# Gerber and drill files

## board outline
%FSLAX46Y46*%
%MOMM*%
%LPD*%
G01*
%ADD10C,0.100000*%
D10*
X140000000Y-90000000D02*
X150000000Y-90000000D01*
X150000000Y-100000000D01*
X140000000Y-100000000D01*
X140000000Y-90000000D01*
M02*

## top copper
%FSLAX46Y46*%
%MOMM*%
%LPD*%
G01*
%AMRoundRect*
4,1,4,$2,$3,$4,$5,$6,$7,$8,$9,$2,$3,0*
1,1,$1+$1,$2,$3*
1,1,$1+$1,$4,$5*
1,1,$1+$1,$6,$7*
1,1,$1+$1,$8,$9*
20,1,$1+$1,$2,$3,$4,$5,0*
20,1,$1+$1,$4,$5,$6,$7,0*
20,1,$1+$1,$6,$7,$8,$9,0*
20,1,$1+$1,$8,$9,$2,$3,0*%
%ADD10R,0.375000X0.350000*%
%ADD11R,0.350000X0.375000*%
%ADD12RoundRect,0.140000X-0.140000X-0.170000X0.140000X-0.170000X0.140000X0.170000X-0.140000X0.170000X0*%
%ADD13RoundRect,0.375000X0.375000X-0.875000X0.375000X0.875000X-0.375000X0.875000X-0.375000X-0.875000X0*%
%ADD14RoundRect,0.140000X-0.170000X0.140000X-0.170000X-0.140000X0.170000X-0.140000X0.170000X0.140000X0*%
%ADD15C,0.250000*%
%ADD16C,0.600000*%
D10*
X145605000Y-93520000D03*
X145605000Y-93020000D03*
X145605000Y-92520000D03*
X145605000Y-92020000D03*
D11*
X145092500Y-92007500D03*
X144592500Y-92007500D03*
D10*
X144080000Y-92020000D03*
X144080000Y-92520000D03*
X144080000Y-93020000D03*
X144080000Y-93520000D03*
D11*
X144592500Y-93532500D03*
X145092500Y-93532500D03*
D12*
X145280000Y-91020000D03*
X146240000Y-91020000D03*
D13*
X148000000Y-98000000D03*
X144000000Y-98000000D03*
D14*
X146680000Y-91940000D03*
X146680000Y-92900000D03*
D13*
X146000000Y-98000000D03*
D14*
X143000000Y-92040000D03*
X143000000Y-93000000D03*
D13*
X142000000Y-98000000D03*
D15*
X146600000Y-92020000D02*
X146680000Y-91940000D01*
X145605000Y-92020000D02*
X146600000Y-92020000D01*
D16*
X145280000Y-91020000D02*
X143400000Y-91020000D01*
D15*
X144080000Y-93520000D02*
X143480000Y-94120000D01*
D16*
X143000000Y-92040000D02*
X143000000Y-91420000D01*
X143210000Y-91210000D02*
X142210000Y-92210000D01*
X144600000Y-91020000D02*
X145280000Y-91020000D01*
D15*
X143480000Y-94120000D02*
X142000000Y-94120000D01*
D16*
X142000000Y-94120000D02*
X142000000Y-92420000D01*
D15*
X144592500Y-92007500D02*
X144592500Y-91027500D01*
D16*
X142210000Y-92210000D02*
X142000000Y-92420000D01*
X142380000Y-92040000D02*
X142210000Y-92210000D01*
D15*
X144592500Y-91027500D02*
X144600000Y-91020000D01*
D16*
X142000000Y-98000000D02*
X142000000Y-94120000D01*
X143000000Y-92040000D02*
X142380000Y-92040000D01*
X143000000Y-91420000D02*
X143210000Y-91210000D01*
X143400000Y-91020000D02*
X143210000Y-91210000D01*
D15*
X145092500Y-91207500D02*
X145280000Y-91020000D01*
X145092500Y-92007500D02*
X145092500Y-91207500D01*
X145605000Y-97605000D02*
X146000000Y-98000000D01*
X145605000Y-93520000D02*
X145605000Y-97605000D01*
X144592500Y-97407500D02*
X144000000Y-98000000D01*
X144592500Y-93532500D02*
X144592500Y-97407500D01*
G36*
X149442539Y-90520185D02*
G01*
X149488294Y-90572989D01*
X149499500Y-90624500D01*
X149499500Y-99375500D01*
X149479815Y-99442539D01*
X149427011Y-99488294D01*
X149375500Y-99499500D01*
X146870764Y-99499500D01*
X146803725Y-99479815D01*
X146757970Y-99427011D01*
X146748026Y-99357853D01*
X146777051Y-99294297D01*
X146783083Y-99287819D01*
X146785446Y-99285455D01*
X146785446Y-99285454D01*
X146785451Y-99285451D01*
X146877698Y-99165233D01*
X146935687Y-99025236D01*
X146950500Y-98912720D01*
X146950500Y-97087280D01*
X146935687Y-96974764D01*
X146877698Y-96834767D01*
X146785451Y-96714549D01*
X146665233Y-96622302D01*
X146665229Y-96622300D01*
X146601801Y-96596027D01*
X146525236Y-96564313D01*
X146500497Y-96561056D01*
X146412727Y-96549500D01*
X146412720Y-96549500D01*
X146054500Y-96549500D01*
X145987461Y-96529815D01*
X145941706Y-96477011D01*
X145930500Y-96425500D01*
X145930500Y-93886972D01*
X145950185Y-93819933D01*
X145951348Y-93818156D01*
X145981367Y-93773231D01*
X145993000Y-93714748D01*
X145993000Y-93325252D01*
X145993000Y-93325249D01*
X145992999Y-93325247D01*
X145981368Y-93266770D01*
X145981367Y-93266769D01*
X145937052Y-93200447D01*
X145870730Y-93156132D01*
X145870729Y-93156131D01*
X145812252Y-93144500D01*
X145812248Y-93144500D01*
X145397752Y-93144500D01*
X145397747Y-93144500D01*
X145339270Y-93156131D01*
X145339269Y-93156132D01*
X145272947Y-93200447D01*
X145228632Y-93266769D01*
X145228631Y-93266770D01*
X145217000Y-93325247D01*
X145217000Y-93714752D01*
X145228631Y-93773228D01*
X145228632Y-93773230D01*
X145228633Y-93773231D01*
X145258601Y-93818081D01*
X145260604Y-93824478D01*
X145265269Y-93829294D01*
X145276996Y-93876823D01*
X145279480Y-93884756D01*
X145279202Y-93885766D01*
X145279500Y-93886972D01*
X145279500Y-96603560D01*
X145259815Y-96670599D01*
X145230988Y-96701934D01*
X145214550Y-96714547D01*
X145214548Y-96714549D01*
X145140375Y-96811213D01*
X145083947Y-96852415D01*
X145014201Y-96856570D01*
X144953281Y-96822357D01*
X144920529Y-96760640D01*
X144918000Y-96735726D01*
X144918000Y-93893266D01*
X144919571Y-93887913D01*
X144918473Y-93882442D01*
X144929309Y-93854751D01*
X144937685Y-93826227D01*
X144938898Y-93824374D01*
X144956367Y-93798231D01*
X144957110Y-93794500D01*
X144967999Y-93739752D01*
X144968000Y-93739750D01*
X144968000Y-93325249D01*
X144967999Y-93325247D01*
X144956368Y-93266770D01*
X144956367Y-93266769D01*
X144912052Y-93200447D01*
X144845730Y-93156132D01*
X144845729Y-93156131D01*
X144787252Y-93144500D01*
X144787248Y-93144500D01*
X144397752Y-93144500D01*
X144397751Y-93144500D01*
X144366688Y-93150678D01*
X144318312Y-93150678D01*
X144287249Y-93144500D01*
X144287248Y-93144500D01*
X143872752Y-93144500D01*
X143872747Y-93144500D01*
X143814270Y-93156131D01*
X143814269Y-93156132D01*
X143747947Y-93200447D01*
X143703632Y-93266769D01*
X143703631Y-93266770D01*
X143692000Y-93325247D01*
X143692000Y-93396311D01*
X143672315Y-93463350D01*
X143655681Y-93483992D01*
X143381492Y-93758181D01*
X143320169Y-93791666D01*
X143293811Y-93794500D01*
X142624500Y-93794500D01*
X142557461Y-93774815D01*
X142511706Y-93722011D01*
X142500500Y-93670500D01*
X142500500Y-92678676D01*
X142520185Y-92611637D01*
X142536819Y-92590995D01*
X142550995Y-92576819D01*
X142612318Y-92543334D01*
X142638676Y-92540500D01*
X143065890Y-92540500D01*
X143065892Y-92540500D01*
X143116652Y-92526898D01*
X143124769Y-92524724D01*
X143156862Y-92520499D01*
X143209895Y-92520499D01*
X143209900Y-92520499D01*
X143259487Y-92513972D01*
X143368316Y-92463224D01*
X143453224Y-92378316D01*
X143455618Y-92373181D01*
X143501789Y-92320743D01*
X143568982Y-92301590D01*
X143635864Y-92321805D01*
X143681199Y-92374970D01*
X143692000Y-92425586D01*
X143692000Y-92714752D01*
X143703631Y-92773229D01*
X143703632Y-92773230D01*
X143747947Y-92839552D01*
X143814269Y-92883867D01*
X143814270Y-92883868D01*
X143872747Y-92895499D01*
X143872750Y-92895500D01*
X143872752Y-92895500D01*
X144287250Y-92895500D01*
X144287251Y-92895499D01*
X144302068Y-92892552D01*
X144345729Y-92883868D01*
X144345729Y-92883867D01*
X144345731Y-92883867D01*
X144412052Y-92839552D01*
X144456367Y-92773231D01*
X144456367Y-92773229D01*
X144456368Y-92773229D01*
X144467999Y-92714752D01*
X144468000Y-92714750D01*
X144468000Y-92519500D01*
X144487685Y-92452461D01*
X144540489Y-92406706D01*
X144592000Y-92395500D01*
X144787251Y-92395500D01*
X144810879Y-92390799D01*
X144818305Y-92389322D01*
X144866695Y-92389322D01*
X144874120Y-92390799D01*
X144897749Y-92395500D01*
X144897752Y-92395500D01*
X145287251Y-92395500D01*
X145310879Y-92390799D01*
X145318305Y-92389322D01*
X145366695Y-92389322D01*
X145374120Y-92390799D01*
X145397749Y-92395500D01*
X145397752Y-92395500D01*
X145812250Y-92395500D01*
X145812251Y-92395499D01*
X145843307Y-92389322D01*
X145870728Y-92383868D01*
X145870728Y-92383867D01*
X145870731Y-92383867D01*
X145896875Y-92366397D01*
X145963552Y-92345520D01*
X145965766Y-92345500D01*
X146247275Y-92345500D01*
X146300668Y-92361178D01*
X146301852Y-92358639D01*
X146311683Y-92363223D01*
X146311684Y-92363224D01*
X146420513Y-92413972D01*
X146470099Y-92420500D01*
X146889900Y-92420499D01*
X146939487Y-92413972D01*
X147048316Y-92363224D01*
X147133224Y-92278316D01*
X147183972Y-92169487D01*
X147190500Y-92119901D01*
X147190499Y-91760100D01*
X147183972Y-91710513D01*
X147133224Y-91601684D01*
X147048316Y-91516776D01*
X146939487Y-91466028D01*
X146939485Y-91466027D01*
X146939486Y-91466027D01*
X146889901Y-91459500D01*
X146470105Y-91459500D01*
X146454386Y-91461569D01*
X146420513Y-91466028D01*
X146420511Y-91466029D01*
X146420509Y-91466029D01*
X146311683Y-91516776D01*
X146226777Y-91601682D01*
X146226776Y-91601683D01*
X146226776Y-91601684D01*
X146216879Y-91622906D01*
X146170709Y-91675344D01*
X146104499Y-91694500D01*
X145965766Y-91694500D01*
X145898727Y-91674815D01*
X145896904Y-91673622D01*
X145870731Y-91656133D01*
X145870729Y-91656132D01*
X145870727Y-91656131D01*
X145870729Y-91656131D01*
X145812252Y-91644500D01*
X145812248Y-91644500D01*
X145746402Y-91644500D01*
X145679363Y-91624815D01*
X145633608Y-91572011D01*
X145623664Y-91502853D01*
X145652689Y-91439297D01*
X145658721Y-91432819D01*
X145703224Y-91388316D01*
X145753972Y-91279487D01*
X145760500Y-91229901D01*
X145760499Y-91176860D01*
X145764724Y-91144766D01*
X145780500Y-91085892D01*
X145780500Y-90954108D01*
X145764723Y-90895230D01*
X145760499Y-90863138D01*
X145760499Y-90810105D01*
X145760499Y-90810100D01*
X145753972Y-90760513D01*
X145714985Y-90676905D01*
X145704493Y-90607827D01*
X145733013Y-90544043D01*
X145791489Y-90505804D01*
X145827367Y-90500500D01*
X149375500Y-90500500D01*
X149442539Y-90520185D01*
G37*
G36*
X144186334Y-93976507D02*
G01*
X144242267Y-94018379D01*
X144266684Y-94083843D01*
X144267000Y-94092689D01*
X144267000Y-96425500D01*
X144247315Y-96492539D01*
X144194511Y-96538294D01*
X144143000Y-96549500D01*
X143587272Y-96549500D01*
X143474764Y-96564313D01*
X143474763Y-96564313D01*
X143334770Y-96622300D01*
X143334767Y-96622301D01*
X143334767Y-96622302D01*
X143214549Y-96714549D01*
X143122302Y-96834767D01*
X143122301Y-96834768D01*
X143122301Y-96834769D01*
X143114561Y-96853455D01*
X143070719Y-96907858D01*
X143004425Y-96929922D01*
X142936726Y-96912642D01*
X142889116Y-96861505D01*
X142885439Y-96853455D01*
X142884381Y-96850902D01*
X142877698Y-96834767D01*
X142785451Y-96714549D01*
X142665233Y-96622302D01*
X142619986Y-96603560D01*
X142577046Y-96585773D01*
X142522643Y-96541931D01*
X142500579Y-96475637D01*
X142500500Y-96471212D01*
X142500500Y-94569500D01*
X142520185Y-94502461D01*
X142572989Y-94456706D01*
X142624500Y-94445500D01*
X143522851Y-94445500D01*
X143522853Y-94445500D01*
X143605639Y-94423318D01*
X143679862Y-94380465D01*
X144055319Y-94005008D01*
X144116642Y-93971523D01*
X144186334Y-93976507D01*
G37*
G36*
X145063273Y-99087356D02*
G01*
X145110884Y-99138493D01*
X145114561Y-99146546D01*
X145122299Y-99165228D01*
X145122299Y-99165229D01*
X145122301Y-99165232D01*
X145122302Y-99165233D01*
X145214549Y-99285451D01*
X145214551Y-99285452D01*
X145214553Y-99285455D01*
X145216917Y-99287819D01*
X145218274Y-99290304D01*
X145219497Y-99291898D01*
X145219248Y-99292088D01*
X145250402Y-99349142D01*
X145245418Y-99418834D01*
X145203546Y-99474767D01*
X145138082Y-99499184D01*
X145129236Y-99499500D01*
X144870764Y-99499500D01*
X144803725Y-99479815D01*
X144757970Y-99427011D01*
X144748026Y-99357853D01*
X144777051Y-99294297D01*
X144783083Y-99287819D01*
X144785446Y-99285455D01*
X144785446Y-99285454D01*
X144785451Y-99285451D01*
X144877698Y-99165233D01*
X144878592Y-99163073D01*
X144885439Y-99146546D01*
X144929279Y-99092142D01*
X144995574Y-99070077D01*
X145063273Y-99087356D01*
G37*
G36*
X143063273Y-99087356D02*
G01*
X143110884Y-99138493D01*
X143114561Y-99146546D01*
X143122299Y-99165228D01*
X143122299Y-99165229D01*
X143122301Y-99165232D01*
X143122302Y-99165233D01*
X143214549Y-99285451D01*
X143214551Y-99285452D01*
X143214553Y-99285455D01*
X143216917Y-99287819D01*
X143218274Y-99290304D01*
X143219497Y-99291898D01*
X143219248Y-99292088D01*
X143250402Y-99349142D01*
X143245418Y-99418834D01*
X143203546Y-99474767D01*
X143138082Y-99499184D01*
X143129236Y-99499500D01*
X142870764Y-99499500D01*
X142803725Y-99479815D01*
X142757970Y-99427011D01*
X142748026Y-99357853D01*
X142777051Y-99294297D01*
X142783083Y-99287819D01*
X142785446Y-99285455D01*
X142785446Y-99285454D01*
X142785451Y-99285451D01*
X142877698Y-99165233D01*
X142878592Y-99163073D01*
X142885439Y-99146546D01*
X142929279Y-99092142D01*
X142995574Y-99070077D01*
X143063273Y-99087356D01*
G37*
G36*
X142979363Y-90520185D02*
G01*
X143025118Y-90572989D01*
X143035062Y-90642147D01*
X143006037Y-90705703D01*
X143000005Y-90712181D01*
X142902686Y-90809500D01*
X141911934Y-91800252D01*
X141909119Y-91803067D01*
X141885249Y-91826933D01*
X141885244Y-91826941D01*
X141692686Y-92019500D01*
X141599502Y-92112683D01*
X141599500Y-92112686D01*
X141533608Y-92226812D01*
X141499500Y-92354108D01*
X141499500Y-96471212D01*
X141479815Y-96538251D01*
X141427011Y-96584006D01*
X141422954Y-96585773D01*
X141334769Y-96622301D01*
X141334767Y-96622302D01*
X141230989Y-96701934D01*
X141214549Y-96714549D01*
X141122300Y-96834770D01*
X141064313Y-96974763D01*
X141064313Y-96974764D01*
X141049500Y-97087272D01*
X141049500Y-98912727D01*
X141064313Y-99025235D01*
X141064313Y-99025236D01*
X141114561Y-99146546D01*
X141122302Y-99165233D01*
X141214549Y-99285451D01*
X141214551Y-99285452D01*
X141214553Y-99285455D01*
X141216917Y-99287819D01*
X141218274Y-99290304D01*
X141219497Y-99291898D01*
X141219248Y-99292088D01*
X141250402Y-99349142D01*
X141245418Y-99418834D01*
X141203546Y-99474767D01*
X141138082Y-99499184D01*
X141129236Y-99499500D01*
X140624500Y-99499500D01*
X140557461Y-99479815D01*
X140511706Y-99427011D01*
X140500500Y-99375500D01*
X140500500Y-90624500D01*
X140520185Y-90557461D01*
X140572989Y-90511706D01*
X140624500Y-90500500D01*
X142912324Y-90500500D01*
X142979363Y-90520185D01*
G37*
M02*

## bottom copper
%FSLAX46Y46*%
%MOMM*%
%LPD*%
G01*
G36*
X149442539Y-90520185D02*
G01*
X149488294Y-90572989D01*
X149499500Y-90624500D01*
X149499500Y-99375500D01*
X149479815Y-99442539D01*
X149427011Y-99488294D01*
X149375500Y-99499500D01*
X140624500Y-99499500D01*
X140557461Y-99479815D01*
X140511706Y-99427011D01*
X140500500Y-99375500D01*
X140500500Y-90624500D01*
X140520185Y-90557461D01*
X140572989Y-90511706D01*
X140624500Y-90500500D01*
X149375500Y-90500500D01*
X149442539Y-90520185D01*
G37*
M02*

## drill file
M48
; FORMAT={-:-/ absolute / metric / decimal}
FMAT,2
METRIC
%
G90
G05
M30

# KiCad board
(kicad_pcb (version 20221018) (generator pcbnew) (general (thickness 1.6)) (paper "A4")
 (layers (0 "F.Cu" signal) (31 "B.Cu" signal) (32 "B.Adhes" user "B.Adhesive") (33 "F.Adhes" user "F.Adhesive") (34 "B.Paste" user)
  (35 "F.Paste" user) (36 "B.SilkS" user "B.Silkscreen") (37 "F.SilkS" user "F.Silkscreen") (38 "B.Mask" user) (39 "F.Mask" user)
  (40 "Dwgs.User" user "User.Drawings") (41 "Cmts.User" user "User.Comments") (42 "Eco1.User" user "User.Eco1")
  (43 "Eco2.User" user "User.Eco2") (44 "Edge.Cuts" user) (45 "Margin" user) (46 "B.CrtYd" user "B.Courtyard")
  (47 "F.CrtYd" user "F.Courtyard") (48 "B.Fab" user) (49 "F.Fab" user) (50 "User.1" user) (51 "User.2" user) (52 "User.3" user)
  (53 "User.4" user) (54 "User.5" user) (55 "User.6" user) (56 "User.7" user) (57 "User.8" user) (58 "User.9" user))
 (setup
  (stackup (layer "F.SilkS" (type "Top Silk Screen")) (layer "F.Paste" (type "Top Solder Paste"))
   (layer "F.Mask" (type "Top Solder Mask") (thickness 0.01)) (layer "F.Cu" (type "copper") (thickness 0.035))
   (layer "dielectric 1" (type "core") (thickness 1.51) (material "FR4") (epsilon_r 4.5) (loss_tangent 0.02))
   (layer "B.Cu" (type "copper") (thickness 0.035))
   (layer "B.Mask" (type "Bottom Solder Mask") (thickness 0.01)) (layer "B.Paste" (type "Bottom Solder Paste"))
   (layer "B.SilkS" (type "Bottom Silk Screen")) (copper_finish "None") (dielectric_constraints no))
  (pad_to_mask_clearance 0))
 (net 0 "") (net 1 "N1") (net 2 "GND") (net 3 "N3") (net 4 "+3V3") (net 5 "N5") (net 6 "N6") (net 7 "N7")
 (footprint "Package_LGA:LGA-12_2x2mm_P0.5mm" (layer "F.Cu") (at 144.8425 92.77 180)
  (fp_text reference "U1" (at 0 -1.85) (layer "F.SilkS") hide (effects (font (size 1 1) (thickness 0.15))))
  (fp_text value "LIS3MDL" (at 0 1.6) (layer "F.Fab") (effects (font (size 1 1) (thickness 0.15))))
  (pad "1" smd rect (at -0.7625 -0.75 180) (size 0.375 0.35) (layers "F.Cu" "F.Paste" "F.Mask") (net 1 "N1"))
  (pad "2" smd rect (at -0.7625 -0.25 180) (size 0.375 0.35) (layers "F.Cu" "F.Paste" "F.Mask") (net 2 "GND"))
  (pad "3" smd rect (at -0.7625 0.25 180) (size 0.375 0.35) (layers "F.Cu" "F.Paste" "F.Mask") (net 2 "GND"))
  (pad "4" smd rect (at -0.7625 0.75 180) (size 0.375 0.35) (layers "F.Cu" "F.Paste" "F.Mask") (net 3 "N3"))
  (pad "5" smd rect (at -0.25 0.7625 270) (size 0.375 0.35) (layers "F.Cu" "F.Paste" "F.Mask") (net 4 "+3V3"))
  (pad "6" smd rect (at 0.25 0.7625 270) (size 0.375 0.35) (layers "F.Cu" "F.Paste" "F.Mask") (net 4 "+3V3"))
  (pad "7" smd rect (at 0.7625 0.75 180) (size 0.375 0.35) (layers "F.Cu" "F.Paste" "F.Mask") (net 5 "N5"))
  (pad "8" smd rect (at 0.7625 0.25 180) (size 0.375 0.35) (layers "F.Cu" "F.Paste" "F.Mask") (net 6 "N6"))
  (pad "9" smd rect (at 0.7625 -0.25 180) (size 0.375 0.35) (layers "F.Cu" "F.Paste" "F.Mask") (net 2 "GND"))
  (pad "10" smd rect (at 0.7625 -0.75 180) (size 0.375 0.35) (layers "F.Cu" "F.Paste" "F.Mask") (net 4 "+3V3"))
  (pad "11" smd rect (at 0.25 -0.7625 270) (size 0.375 0.35) (layers "F.Cu" "F.Paste" "F.Mask") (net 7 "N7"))
  (pad "12" smd rect (at -0.25 -0.7625 270) (size 0.375 0.35) (layers "F.Cu" "F.Paste" "F.Mask") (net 2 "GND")))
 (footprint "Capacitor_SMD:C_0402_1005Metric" (layer "F.Cu") (at 145.76 91.02)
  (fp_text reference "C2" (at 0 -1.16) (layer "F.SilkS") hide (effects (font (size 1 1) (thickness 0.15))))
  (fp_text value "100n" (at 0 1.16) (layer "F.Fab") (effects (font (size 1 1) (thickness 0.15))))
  (pad "1" smd roundrect (at -0.48 0) (size 0.56 0.62) (layers "F.Cu" "F.Paste" "F.Mask") (roundrect_rratio 0.25) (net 4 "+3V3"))
  (pad "2" smd roundrect (at 0.48 0) (size 0.56 0.62) (layers "F.Cu" "F.Paste" "F.Mask") (roundrect_rratio 0.25) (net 2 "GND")))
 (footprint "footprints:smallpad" (layer "F.Cu") (at 148 98 90)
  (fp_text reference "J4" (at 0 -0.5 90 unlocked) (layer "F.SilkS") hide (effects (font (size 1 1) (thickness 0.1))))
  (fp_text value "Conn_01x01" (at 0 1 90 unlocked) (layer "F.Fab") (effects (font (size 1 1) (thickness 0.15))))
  (pad "1" smd roundrect (at 0 0 90) (size 2.5 1.5) (layers "F.Cu" "F.Paste" "F.Mask") (roundrect_rratio 0.25) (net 2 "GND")))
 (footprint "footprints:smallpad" (layer "F.Cu") (at 144 98 90)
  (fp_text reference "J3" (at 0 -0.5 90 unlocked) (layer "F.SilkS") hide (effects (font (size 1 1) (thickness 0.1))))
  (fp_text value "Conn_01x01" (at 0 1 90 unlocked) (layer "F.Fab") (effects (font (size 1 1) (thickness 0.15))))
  (pad "1" smd roundrect (at 0 0 90) (size 2.5 1.5) (layers "F.Cu" "F.Paste" "F.Mask") (roundrect_rratio 0.25) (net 7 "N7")))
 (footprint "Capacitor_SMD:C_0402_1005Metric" (layer "F.Cu") (at 146.68 92.42 -90)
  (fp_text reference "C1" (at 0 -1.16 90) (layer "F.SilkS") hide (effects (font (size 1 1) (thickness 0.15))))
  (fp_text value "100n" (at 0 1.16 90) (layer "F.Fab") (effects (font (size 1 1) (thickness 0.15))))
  (pad "1" smd roundrect (at -0.48 0 270) (size 0.56 0.62) (layers "F.Cu" "F.Paste" "F.Mask") (roundrect_rratio 0.25) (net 3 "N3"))
  (pad "2" smd roundrect (at 0.48 0 270) (size 0.56 0.62) (layers "F.Cu" "F.Paste" "F.Mask") (roundrect_rratio 0.25) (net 2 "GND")))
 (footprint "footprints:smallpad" (layer "F.Cu") (at 146 98 90)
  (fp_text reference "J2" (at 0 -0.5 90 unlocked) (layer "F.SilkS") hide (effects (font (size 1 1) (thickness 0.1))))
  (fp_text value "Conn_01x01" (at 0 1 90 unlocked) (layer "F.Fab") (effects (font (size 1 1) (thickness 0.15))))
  (pad "1" smd roundrect (at 0 0 90) (size 2.5 1.5) (layers "F.Cu" "F.Paste" "F.Mask") (roundrect_rratio 0.25) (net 1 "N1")))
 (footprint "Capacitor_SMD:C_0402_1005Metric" (layer "F.Cu") (at 143 92.52 -90)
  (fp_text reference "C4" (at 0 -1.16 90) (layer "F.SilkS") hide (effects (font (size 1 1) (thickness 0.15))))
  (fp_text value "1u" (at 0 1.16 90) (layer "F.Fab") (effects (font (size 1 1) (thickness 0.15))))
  (pad "1" smd roundrect (at -0.48 0 270) (size 0.56 0.62) (layers "F.Cu" "F.Paste" "F.Mask") (roundrect_rratio 0.25) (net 4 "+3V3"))
  (pad "2" smd roundrect (at 0.48 0 270) (size 0.56 0.62) (layers "F.Cu" "F.Paste" "F.Mask") (roundrect_rratio 0.25) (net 2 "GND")))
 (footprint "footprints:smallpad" (layer "F.Cu") (at 142 98 90)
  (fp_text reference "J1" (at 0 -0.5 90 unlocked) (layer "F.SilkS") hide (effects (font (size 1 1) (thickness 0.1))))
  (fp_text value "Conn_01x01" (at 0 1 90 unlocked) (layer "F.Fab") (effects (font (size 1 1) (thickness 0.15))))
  (pad "1" smd roundrect (at 0 0 90) (size 2.5 1.5) (layers "F.Cu" "F.Paste" "F.Mask") (roundrect_rratio 0.25) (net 4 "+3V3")))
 (gr_rect (start 140 90) (end 150 100) (stroke (width 0.1) (type default)) (fill none) (layer "Edge.Cuts"))
 (segment (start 146.6 92.02) (end 146.68 91.94) (width 0.25) (layer "F.Cu") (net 3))
 (segment (start 145.605 92.02) (end 146.6 92.02) (width 0.25) (layer "F.Cu") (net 3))
 (segment (start 145.28 91.02) (end 143.4 91.02) (width 0.6) (layer "F.Cu") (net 4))
 (segment (start 144.08 93.52) (end 143.48 94.12) (width 0.25) (layer "F.Cu") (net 4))
 (segment (start 143 92.04) (end 143 91.42) (width 0.6) (layer "F.Cu") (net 4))
 (segment (start 143.21 91.21) (end 142.21 92.21) (width 0.6) (layer "F.Cu") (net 4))
 (segment (start 144.6 91.02) (end 145.28 91.02) (width 0.6) (layer "F.Cu") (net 4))
 (segment (start 143.48 94.12) (end 142 94.12) (width 0.25) (layer "F.Cu") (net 4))
 (segment (start 142 94.12) (end 142 92.42) (width 0.6) (layer "F.Cu") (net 4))
 (segment (start 144.5925 92.0075) (end 144.5925 91.0275) (width 0.25) (layer "F.Cu") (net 4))
 (segment (start 142.21 92.21) (end 142 92.42) (width 0.6) (layer "F.Cu") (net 4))
 (segment (start 142.38 92.04) (end 142.21 92.21) (width 0.6) (layer "F.Cu") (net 4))
 (segment (start 144.5925 91.0275) (end 144.6 91.02) (width 0.25) (layer "F.Cu") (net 4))
 (segment (start 142 98) (end 142 94.12) (width 0.6) (layer "F.Cu") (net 4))
 (segment (start 143 92.04) (end 142.38 92.04) (width 0.6) (layer "F.Cu") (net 4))
 (segment (start 143 91.42) (end 143.21 91.21) (width 0.6) (layer "F.Cu") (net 4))
 (segment (start 143.4 91.02) (end 143.21 91.21) (width 0.6) (layer "F.Cu") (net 4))
 (segment (start 145.0925 91.2075) (end 145.28 91.02) (width 0.25) (layer "F.Cu") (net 4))
 (segment (start 145.0925 92.0075) (end 145.0925 91.2075) (width 0.25) (layer "F.Cu") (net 4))
 (segment (start 145.605 97.605) (end 146 98) (width 0.25) (layer "F.Cu") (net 1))
 (segment (start 145.605 93.52) (end 145.605 97.605) (width 0.25) (layer "F.Cu") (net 1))
 (segment (start 144.5925 97.4075) (end 144 98) (width 0.25) (layer "F.Cu") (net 7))
 (segment (start 144.5925 93.5325) (end 144.5925 97.4075) (width 0.25) (layer "F.Cu") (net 7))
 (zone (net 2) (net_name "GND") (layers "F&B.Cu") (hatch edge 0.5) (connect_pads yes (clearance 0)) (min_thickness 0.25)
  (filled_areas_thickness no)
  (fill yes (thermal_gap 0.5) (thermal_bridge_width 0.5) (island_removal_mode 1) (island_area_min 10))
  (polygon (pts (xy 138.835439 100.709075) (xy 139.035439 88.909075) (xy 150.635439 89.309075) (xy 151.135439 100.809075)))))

